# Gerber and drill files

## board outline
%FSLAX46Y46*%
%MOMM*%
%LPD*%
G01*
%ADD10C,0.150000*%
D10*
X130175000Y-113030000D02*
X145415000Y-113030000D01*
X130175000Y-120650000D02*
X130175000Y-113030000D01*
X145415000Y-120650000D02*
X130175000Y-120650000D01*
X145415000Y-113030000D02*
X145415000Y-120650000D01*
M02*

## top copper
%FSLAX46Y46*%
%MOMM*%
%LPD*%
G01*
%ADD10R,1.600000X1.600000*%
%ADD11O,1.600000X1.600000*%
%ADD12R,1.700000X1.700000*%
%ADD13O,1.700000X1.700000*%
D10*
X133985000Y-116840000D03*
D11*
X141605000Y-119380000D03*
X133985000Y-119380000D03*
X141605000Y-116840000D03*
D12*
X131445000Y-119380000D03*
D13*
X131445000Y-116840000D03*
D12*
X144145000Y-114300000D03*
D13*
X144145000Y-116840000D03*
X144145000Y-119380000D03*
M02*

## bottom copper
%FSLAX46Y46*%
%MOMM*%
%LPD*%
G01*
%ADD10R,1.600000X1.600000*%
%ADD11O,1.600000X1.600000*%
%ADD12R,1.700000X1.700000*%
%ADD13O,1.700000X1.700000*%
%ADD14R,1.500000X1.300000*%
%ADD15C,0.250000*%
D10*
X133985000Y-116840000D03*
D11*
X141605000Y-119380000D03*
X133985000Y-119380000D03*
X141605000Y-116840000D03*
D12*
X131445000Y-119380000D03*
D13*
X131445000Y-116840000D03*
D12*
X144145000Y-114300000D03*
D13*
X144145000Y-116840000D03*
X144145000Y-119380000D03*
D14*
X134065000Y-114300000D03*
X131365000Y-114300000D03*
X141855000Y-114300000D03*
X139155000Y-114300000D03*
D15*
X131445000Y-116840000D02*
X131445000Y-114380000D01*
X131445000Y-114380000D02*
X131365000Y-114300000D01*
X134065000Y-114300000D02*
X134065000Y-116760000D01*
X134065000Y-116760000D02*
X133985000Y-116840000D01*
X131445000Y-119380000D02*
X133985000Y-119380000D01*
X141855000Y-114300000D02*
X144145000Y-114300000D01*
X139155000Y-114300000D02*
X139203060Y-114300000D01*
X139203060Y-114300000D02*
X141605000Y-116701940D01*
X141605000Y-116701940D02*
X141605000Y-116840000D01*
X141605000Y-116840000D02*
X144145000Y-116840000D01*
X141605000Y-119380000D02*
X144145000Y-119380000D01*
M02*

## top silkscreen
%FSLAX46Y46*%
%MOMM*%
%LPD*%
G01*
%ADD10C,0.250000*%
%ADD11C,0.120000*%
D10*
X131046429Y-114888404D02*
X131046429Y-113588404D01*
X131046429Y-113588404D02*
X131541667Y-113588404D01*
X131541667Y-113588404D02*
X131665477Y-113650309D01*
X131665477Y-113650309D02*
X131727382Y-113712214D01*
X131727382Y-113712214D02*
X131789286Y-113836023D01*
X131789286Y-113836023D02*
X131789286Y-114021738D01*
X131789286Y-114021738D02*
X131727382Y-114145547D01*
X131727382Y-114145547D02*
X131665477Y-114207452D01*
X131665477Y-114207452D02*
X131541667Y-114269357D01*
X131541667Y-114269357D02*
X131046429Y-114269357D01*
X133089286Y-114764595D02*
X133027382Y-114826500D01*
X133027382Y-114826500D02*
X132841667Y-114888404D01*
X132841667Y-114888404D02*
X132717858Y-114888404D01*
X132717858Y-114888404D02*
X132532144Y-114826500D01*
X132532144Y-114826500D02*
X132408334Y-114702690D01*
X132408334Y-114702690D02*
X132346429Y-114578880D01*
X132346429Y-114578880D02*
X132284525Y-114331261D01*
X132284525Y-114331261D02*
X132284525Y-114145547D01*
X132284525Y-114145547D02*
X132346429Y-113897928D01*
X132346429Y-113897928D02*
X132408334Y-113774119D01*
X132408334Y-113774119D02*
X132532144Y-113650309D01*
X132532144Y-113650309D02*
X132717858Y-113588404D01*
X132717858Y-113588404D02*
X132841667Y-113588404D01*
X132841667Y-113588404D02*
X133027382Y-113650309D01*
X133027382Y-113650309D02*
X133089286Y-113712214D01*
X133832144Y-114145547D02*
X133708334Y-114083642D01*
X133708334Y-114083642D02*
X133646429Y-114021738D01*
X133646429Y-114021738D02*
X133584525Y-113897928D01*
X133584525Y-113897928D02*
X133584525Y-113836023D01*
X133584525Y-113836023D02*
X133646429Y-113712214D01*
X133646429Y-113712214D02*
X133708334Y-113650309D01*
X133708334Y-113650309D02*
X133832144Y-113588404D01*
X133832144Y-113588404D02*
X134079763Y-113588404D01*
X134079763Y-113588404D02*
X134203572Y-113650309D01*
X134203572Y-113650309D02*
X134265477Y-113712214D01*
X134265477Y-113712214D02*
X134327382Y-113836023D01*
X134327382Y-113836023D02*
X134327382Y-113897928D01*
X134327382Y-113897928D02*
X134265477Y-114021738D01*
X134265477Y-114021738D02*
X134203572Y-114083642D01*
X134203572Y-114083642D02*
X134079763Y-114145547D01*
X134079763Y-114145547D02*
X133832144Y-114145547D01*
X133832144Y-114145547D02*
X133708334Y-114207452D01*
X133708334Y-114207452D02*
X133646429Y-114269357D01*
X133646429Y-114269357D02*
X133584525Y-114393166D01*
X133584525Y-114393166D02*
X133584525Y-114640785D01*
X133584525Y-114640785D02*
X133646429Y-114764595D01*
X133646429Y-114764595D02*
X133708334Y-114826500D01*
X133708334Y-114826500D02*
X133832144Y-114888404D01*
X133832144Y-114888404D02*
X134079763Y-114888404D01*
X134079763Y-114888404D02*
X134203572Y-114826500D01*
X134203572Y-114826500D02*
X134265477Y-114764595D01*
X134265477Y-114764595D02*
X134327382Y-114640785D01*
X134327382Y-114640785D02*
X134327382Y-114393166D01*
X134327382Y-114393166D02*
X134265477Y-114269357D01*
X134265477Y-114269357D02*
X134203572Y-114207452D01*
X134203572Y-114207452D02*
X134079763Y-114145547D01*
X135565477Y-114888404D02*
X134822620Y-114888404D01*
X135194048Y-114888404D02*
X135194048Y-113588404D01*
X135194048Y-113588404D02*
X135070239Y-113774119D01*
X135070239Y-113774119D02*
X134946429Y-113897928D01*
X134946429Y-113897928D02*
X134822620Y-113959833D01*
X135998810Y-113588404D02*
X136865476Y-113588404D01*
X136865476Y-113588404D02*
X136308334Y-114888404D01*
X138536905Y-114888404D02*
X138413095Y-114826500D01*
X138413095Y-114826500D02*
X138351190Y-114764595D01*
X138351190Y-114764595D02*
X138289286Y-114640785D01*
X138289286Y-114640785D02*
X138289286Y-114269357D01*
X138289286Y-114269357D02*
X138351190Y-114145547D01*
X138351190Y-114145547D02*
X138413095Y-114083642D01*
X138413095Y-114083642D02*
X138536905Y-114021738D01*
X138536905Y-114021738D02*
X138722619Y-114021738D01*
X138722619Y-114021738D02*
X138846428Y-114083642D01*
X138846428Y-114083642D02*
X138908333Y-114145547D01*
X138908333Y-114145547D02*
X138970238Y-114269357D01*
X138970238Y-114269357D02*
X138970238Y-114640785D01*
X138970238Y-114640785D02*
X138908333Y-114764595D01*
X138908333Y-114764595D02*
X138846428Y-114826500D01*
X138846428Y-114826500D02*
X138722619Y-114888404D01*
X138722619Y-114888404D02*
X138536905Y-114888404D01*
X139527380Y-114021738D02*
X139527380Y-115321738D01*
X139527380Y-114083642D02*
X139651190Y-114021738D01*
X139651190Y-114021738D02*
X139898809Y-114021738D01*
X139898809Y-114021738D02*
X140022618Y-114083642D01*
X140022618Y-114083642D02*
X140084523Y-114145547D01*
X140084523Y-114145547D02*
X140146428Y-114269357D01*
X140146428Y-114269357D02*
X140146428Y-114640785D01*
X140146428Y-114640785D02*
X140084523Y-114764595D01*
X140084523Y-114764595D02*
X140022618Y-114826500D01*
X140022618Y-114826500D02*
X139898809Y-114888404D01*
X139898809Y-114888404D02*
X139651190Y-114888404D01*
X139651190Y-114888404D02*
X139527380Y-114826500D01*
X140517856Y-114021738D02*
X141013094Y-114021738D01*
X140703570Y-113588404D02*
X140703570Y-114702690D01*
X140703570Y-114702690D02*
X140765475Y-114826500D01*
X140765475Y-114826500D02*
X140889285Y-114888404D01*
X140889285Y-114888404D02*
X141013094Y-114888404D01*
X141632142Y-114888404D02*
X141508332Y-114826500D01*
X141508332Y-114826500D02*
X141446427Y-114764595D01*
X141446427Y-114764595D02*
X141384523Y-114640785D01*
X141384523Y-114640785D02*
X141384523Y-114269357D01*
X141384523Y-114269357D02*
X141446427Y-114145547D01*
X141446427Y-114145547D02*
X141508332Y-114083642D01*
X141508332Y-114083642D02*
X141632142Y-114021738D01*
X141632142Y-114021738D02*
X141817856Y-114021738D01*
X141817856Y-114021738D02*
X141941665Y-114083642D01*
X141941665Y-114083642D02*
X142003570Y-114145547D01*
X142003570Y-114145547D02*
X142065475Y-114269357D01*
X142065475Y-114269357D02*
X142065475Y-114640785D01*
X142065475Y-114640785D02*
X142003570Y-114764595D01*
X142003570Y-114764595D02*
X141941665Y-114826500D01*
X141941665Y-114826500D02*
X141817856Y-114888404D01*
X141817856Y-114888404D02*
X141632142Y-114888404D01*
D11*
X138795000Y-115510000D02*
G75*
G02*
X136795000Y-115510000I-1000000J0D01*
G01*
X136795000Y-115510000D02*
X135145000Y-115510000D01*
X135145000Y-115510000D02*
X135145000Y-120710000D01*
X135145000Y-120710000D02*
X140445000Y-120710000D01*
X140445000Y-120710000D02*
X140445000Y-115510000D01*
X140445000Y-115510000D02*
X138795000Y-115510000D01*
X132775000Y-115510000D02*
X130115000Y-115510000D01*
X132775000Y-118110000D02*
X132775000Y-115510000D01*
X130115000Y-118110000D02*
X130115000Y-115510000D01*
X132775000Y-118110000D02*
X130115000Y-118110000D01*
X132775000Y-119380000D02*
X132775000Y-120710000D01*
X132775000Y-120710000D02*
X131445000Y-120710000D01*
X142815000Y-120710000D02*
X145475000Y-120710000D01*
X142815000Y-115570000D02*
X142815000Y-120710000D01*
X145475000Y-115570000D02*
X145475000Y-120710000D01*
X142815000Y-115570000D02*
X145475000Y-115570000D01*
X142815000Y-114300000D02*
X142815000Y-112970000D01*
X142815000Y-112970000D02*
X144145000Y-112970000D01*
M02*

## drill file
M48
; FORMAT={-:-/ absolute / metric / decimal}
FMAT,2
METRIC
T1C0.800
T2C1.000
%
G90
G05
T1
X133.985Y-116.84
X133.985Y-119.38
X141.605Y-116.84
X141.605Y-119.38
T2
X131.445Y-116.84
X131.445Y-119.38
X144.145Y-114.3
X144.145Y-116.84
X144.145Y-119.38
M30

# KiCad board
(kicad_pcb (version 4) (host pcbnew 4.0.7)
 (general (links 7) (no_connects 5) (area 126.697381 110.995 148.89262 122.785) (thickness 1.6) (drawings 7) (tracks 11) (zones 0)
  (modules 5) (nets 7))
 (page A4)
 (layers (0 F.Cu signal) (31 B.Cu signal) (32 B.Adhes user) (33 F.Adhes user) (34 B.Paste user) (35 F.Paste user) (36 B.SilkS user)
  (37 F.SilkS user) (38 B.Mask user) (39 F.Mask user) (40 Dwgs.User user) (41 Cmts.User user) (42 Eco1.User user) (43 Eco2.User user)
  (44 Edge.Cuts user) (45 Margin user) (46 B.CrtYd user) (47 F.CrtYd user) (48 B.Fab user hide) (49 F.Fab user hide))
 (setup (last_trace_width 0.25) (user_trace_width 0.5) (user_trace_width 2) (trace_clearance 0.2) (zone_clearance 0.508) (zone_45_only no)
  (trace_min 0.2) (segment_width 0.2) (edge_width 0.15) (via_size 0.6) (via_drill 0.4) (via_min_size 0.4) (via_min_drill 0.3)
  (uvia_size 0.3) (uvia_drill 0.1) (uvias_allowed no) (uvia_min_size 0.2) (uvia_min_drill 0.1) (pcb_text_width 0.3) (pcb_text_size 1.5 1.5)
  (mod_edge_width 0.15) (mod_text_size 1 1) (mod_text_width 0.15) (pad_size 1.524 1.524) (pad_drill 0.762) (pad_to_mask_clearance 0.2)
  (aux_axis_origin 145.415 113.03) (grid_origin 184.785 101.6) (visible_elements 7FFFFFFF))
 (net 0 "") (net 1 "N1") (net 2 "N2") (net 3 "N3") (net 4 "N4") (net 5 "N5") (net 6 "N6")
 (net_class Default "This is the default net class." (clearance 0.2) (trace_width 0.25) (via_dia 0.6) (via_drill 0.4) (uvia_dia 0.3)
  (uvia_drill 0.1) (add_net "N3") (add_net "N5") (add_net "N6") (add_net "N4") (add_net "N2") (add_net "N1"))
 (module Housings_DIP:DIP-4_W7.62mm (layer F.Cu) (at 133.985 116.84)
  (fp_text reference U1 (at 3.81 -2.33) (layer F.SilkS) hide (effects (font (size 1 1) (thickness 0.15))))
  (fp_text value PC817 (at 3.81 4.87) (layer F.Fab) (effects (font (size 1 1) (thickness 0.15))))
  (fp_arc (start 3.81 -1.33) (end 2.81 -1.33) (angle -180) (layer F.SilkS) (width 0.12))
  (fp_line (start 2.81 -1.33) (end 1.16 -1.33) (layer F.SilkS) (width 0.12))
  (fp_line (start 1.16 -1.33) (end 1.16 3.87) (layer F.SilkS) (width 0.12))
  (fp_line (start 1.16 3.87) (end 6.46 3.87) (layer F.SilkS) (width 0.12))
  (fp_line (start 6.46 3.87) (end 6.46 -1.33) (layer F.SilkS) (width 0.12))
  (fp_line (start 6.46 -1.33) (end 4.81 -1.33) (layer F.SilkS) (width 0.12))
  (pad 1 thru_hole rect (at 0 0) (size 1.6 1.6) (drill 0.8) (layers *.Cu *.Mask) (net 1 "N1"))
  (pad 3 thru_hole oval (at 7.62 2.54) (size 1.6 1.6) (drill 0.8) (layers *.Cu *.Mask) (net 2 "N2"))
  (pad 2 thru_hole oval (at 0 2.54) (size 1.6 1.6) (drill 0.8) (layers *.Cu *.Mask) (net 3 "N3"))
  (pad 4 thru_hole oval (at 7.62 0) (size 1.6 1.6) (drill 0.8) (layers *.Cu *.Mask) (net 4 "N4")))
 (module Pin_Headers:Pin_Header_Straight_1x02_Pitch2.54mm (layer F.Cu) (at 131.445 119.38 180)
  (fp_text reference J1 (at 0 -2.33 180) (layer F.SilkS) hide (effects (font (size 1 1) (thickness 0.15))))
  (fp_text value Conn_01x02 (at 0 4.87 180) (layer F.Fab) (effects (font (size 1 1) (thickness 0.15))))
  (fp_line (start -1.33 3.87) (end 1.33 3.87) (layer F.SilkS) (width 0.12))
  (fp_line (start -1.33 1.27) (end -1.33 3.87) (layer F.SilkS) (width 0.12))
  (fp_line (start 1.33 1.27) (end 1.33 3.87) (layer F.SilkS) (width 0.12))
  (fp_line (start -1.33 1.27) (end 1.33 1.27) (layer F.SilkS) (width 0.12))
  (fp_line (start -1.33 0) (end -1.33 -1.33) (layer F.SilkS) (width 0.12))
  (fp_line (start -1.33 -1.33) (end 0 -1.33) (layer F.SilkS) (width 0.12))
  (pad 1 thru_hole rect (at 0 0 180) (size 1.7 1.7) (drill 1) (layers *.Cu *.Mask) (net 3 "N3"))
  (pad 2 thru_hole oval (at 0 2.54 180) (size 1.7 1.7) (drill 1) (layers *.Cu *.Mask) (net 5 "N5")))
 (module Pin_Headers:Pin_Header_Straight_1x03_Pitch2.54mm (layer F.Cu) (at 144.145 114.3)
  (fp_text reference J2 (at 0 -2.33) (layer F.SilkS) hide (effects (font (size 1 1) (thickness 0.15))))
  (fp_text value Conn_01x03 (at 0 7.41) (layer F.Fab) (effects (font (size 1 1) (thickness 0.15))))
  (fp_line (start -1.33 6.41) (end 1.33 6.41) (layer F.SilkS) (width 0.12))
  (fp_line (start -1.33 1.27) (end -1.33 6.41) (layer F.SilkS) (width 0.12))
  (fp_line (start 1.33 1.27) (end 1.33 6.41) (layer F.SilkS) (width 0.12))
  (fp_line (start -1.33 1.27) (end 1.33 1.27) (layer F.SilkS) (width 0.12))
  (fp_line (start -1.33 0) (end -1.33 -1.33) (layer F.SilkS) (width 0.12))
  (fp_line (start -1.33 -1.33) (end 0 -1.33) (layer F.SilkS) (width 0.12))
  (pad 1 thru_hole rect (at 0 0) (size 1.7 1.7) (drill 1) (layers *.Cu *.Mask) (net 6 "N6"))
  (pad 2 thru_hole oval (at 0 2.54) (size 1.7 1.7) (drill 1) (layers *.Cu *.Mask) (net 4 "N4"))
  (pad 3 thru_hole oval (at 0 5.08) (size 1.7 1.7) (drill 1) (layers *.Cu *.Mask) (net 2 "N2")))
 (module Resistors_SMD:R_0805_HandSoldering (layer B.Cu) (at 132.715 114.3 180)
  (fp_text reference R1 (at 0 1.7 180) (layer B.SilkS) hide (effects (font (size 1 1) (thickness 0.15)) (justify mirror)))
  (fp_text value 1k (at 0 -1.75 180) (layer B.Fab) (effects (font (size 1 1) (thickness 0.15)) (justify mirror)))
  (pad 1 smd rect (at -1.35 0 180) (size 1.5 1.3) (layers B.Cu B.Paste B.Mask) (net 1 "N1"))
  (pad 2 smd rect (at 1.35 0 180) (size 1.5 1.3) (layers B.Cu B.Paste B.Mask) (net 5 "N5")))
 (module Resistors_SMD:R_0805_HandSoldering (layer B.Cu) (at 140.505 114.3 180)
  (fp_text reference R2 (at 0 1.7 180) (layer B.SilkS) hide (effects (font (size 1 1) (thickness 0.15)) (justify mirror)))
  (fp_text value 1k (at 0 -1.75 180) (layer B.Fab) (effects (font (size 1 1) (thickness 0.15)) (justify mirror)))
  (pad 1 smd rect (at -1.35 0 180) (size 1.5 1.3) (layers B.Cu B.Paste B.Mask) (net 6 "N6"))
  (pad 2 smd rect (at 1.35 0 180) (size 1.5 1.3) (layers B.Cu B.Paste B.Mask) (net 4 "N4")))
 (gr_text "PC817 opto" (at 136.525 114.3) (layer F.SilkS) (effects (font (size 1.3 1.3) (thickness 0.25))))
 (gr_line (start 130.175 113.03) (end 145.415 113.03) (layer Edge.Cuts) (width 0.15))
 (gr_line (start 130.175 120.65) (end 130.175 113.03) (layer Edge.Cuts) (width 0.15))
 (gr_line (start 145.415 120.65) (end 130.175 120.65) (layer Edge.Cuts) (width 0.15))
 (gr_line (start 145.415 113.03) (end 145.415 120.65) (layer Edge.Cuts) (width 0.15))
 (segment (start 131.445 116.84) (end 131.445 114.38) (width 0.25) (layer B.Cu) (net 5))
 (segment (start 131.445 114.38) (end 131.365 114.3) (width 0.25) (layer B.Cu) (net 5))
 (segment (start 134.065 114.3) (end 134.065 116.76) (width 0.25) (layer B.Cu) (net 1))
 (segment (start 134.065 116.76) (end 133.985 116.84) (width 0.25) (layer B.Cu) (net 1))
 (segment (start 131.445 119.38) (end 133.985 119.38) (width 0.25) (layer B.Cu) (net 3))
 (segment (start 141.855 114.3) (end 144.145 114.3) (width 0.25) (layer B.Cu) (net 6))
 (segment (start 139.155 114.3) (end 139.20306 114.3) (width 0.25) (layer B.Cu) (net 4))
 (segment (start 139.20306 114.3) (end 141.605 116.70194) (width 0.25) (layer B.Cu) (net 4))
 (segment (start 141.605 116.70194) (end 141.605 116.84) (width 0.25) (layer B.Cu) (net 4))
 (segment (start 141.605 116.84) (end 144.145 116.84) (width 0.25) (layer B.Cu) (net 4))
 (segment (start 141.605 119.38) (end 144.145 119.38) (width 0.25) (layer B.Cu) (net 2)))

